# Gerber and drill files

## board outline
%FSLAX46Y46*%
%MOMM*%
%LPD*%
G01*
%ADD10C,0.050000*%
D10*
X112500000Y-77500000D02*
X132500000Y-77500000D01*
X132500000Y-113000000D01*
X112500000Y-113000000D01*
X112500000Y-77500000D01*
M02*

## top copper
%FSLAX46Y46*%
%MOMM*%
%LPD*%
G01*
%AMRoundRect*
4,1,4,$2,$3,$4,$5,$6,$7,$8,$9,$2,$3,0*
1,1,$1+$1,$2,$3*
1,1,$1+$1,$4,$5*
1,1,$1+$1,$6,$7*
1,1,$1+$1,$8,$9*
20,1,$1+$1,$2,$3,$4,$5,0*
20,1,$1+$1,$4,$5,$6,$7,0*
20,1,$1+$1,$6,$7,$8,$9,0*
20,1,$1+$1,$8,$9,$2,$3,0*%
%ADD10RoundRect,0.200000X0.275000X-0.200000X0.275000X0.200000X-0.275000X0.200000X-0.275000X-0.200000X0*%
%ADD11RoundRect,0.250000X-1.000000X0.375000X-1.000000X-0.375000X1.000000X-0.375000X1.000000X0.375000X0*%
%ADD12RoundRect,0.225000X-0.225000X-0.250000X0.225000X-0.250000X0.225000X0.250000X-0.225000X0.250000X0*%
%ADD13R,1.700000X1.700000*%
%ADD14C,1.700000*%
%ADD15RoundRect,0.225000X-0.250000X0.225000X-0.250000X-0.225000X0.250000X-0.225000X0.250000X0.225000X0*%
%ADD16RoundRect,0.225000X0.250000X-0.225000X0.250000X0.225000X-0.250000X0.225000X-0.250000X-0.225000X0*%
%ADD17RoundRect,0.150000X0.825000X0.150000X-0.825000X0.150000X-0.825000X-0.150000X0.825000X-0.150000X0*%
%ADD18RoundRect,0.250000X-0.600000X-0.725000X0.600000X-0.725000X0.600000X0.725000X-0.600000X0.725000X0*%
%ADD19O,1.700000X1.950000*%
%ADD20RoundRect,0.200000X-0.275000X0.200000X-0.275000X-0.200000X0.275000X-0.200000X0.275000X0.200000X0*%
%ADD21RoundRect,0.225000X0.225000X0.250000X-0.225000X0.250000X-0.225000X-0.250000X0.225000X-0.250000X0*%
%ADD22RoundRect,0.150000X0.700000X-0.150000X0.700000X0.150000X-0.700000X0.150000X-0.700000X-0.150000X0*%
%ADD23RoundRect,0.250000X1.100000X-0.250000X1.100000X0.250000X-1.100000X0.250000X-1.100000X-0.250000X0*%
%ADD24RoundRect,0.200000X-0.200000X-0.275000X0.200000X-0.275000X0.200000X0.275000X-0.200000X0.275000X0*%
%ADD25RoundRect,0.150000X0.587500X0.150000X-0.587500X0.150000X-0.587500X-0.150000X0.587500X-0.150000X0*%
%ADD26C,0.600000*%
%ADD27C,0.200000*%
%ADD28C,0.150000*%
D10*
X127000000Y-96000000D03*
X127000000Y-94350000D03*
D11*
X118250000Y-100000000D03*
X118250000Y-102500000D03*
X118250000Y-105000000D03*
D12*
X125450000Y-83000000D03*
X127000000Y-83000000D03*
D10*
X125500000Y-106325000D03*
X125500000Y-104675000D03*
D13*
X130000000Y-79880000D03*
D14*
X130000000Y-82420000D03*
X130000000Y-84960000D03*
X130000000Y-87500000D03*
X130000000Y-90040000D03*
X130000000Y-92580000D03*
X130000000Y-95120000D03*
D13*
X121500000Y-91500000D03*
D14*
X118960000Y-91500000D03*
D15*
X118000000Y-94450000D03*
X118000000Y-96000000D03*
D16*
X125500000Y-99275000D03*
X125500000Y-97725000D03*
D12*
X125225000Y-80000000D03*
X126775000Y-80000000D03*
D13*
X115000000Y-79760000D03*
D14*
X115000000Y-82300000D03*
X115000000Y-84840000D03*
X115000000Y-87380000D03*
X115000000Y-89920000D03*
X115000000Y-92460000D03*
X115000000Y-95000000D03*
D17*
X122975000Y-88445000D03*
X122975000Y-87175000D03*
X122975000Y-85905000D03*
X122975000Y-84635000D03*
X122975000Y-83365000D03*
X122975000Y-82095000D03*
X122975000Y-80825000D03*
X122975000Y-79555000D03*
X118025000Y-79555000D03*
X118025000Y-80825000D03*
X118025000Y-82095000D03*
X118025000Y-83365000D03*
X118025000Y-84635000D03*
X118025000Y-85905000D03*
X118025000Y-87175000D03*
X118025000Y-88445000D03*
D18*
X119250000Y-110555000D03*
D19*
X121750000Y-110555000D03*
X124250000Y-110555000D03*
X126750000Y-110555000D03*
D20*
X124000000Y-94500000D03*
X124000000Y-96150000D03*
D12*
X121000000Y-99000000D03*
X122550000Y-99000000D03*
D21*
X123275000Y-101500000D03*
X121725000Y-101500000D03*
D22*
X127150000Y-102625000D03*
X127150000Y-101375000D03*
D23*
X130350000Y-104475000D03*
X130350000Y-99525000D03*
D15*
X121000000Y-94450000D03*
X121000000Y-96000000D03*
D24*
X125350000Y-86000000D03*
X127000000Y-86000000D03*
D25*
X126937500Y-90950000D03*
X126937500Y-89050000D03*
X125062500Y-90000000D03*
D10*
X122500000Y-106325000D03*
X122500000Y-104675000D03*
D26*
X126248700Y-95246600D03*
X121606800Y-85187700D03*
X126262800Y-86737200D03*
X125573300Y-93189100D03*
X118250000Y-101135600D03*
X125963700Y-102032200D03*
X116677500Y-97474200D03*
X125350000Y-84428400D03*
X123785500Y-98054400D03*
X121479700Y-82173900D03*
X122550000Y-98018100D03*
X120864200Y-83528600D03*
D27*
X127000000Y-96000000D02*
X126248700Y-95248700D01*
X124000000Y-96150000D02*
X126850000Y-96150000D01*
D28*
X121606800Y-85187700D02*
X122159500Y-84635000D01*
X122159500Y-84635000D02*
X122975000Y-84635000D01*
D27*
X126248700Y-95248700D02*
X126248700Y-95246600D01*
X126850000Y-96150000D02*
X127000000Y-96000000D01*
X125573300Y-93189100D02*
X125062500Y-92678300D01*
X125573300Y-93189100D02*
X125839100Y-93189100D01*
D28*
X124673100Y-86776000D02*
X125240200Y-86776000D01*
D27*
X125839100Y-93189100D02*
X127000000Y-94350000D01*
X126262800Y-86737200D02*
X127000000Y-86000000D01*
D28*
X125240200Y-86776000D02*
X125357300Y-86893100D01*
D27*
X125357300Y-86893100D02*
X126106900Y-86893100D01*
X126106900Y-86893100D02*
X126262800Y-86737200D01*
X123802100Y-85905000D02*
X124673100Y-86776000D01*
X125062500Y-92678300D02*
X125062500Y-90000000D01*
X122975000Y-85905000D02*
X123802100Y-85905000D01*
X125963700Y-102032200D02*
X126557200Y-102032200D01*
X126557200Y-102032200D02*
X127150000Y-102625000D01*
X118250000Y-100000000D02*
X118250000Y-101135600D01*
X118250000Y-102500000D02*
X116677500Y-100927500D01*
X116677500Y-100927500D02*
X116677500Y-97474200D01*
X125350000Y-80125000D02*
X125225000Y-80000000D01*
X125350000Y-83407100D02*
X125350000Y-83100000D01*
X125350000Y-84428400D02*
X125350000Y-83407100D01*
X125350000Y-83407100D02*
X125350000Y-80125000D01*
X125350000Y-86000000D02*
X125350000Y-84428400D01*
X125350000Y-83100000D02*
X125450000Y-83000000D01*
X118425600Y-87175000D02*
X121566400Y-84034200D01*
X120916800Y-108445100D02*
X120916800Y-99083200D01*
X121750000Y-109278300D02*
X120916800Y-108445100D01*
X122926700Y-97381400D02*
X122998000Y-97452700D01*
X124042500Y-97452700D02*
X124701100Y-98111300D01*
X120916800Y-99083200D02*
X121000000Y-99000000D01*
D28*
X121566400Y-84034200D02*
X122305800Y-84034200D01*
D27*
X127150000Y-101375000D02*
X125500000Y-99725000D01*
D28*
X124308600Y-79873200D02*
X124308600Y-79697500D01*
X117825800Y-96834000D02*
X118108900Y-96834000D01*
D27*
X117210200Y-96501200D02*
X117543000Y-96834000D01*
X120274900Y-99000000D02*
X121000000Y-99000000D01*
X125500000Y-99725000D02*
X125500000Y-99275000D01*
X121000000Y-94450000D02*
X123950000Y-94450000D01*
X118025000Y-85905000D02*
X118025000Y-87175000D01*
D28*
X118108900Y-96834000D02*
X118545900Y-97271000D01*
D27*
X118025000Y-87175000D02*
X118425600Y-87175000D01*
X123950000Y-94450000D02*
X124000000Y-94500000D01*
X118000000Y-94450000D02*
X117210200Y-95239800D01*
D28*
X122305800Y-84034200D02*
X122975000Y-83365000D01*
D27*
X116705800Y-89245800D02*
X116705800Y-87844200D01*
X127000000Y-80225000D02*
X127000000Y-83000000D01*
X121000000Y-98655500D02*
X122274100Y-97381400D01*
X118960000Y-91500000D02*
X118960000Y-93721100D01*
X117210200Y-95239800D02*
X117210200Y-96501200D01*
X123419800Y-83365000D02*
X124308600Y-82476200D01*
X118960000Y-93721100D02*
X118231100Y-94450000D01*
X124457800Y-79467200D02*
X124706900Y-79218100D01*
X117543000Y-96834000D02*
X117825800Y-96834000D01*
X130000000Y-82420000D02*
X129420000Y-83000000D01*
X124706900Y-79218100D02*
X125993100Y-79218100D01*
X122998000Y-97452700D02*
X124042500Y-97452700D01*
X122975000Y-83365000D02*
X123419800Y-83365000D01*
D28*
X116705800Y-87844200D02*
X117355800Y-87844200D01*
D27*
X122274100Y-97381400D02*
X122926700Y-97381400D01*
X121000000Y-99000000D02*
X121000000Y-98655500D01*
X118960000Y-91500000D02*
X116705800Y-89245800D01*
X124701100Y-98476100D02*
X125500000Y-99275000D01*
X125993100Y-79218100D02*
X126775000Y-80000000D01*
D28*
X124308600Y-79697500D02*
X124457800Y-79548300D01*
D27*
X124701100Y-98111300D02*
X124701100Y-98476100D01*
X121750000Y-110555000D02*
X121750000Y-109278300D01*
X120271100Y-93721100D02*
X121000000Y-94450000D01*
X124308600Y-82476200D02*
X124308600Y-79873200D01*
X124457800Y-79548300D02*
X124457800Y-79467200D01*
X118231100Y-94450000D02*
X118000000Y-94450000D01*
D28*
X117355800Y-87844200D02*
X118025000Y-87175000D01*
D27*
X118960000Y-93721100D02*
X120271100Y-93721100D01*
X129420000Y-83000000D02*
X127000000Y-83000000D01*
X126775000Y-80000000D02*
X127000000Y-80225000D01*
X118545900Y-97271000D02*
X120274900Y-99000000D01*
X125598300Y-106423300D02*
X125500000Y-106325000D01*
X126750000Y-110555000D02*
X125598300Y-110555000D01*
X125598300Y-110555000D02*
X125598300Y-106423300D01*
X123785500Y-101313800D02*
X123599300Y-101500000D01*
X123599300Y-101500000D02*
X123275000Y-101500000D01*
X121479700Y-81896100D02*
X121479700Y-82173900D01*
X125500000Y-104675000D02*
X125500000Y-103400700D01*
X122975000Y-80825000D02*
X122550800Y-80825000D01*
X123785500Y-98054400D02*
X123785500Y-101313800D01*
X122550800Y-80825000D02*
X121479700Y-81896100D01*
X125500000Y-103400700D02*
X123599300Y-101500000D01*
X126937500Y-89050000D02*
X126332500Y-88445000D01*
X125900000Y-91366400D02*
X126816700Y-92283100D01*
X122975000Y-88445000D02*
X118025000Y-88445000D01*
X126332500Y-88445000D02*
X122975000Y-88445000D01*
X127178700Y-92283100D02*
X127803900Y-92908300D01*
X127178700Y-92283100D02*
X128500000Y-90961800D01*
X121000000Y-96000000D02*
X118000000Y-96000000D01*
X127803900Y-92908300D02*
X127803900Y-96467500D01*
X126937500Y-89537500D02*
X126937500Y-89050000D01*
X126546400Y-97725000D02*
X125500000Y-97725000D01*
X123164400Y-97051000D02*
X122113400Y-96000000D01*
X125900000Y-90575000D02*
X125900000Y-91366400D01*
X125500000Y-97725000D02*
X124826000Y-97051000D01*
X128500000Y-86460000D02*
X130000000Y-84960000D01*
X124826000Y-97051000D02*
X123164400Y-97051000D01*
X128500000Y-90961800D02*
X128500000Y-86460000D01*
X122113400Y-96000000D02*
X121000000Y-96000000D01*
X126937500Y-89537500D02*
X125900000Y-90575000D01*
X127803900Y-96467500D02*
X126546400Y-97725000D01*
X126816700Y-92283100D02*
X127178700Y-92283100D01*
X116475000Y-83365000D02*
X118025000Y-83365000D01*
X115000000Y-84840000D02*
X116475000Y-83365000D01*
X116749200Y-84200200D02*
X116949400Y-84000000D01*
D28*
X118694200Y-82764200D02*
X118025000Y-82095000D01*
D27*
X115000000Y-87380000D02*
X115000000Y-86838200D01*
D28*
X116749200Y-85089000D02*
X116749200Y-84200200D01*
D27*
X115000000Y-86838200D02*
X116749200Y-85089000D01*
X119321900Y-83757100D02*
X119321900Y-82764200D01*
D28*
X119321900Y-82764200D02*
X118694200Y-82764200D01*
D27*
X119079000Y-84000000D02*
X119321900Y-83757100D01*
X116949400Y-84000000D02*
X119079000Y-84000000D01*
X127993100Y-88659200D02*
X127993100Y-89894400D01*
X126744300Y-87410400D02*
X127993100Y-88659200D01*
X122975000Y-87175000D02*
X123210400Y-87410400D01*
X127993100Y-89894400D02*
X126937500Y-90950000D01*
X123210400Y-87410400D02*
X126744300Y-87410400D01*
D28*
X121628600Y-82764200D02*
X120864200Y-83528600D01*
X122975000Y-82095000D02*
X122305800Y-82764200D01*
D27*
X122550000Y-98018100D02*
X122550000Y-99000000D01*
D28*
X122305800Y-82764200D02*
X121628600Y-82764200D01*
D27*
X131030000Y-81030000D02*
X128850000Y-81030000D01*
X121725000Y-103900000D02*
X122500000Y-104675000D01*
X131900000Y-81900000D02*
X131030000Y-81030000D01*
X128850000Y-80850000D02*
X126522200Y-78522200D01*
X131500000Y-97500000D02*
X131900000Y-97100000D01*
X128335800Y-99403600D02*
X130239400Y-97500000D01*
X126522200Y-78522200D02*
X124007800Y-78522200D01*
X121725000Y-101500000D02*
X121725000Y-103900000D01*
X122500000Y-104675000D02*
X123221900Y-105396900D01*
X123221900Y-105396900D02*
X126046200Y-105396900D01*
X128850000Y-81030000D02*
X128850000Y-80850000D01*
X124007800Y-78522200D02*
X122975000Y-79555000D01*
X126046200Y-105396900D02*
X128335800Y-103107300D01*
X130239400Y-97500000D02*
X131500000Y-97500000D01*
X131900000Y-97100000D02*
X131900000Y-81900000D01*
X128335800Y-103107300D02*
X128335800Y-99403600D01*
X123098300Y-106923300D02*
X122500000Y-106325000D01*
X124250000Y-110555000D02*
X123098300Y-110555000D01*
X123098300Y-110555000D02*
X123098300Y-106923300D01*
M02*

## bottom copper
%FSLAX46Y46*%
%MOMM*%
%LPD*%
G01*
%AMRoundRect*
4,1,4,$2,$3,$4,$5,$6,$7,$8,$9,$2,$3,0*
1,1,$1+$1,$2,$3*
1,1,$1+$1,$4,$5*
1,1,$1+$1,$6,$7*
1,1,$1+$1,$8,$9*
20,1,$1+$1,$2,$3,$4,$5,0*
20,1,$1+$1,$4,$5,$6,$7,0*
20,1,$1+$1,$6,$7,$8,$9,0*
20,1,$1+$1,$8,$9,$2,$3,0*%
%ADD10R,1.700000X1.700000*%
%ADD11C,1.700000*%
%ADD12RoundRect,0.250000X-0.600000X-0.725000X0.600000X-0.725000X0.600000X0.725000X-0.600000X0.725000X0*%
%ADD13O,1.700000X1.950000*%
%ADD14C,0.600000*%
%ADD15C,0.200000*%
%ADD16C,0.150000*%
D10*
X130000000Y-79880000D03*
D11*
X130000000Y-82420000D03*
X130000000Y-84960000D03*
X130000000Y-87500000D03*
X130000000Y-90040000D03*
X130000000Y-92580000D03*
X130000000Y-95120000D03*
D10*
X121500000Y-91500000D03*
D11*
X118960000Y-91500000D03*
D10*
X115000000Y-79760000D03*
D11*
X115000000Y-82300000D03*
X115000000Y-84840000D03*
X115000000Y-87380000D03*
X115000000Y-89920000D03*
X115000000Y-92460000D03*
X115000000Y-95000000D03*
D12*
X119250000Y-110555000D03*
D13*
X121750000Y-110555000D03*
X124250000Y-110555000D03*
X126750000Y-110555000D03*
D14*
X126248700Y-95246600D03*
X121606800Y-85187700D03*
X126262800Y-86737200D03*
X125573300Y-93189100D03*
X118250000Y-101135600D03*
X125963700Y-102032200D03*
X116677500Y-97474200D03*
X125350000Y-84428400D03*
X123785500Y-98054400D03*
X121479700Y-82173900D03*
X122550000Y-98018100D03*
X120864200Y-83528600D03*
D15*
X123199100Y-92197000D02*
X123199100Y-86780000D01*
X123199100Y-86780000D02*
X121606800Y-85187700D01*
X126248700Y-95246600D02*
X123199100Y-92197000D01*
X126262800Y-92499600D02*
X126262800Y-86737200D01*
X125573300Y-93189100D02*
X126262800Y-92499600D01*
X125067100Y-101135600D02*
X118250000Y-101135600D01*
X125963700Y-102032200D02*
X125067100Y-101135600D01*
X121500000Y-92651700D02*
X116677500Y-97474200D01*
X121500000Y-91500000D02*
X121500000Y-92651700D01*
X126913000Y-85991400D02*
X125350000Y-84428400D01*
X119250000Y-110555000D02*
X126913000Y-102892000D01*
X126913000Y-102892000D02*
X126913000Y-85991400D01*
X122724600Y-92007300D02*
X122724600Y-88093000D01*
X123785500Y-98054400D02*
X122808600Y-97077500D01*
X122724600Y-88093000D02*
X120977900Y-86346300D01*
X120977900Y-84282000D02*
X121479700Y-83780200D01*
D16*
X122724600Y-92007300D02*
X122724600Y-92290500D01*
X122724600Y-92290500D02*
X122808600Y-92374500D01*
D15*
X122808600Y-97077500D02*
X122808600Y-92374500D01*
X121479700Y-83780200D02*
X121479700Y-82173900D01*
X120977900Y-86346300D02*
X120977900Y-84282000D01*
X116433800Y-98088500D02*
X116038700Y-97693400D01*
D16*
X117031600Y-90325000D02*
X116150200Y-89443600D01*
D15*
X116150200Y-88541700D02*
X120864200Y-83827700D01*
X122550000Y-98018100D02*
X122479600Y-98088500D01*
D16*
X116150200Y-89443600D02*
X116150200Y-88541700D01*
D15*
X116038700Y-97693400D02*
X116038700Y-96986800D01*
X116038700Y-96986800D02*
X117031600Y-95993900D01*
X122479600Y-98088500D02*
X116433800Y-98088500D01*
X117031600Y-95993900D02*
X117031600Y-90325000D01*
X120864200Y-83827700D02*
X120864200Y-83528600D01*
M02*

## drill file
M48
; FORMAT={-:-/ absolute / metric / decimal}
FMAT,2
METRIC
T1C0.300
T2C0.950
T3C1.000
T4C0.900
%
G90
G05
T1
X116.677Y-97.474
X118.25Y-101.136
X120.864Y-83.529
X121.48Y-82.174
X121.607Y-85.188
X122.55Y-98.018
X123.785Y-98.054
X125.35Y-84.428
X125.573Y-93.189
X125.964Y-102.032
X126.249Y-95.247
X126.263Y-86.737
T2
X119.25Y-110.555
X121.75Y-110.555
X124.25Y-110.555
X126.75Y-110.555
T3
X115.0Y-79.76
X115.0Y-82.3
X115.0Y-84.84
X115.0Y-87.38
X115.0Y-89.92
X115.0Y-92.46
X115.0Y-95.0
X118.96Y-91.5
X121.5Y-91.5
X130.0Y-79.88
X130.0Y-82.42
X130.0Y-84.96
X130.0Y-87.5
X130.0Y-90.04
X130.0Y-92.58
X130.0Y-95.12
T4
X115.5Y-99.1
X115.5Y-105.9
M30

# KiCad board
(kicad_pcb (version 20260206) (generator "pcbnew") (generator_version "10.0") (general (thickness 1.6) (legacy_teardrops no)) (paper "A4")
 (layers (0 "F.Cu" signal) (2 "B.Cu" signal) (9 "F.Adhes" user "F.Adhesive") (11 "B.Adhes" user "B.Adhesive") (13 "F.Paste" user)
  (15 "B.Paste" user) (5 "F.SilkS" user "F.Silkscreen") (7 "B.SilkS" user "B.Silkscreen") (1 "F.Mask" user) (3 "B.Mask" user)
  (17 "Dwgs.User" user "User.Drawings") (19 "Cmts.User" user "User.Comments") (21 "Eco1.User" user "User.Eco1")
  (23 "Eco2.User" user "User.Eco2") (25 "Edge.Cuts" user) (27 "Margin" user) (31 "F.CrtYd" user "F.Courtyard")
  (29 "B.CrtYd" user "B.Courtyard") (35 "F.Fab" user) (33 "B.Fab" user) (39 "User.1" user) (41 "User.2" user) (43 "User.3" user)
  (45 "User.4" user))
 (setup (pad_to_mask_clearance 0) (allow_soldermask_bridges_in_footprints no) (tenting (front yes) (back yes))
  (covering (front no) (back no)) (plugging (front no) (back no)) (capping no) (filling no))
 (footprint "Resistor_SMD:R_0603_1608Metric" (layer "F.Cu") (at 127 95.175 90)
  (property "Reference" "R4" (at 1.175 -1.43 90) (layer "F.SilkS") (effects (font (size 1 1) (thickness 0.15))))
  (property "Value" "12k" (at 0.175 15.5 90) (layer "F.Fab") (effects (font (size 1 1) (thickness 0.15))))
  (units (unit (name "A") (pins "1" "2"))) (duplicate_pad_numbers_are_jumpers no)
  (pad "1" smd roundrect (at -0.825 0 90) (size 0.8 0.95) (layers "F.Cu" "F.Mask" "F.Paste") (roundrect_rratio 0.25) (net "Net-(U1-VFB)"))
  (pad "2" smd roundrect (at 0.825 0 90) (size 0.8 0.95) (layers "F.Cu" "F.Mask" "F.Paste") (roundrect_rratio 0.25) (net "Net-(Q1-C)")))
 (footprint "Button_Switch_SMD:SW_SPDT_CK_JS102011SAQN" (layer "F.Cu") (at 115.5 102.5 -90)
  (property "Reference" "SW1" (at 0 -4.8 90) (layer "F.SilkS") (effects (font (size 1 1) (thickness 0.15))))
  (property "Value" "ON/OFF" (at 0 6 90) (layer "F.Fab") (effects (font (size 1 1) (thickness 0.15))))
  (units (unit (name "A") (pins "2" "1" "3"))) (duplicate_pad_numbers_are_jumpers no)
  (pad "" np_thru_hole circle (at -3.4 0 270) (size 0.9 0.9) (drill 0.9) (layers "*.Cu" "*.Mask"))
  (pad "" np_thru_hole circle (at 3.4 0 270) (size 0.9 0.9) (drill 0.9) (layers "*.Cu" "*.Mask"))
  (pad "1" smd roundrect (at -2.5 -2.75 270) (size 1.25 2.5) (layers "F.Cu" "F.Mask" "F.Paste") (roundrect_rratio 0.2) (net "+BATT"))
  (pad "2" smd roundrect (at 0 -2.75 270) (size 1.25 2.5) (layers "F.Cu" "F.Mask" "F.Paste") (roundrect_rratio 0.2) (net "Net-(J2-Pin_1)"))
  (pad "3" smd roundrect (at 2.5 -2.75 270) (size 1.25 2.5) (layers "F.Cu" "F.Mask" "F.Paste") (roundrect_rratio 0.2)
   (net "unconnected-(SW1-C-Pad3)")))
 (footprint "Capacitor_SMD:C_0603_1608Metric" (layer "F.Cu") (at 126.225 83)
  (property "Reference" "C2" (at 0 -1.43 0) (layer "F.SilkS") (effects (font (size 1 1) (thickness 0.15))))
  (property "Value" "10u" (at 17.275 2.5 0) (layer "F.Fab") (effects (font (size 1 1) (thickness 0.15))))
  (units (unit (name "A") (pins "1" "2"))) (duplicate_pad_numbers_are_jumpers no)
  (pad "1" smd roundrect (at -0.775 0) (size 0.9 0.95) (layers "F.Cu" "F.Mask" "F.Paste") (roundrect_rratio 0.25) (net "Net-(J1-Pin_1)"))
  (pad "2" smd roundrect (at 0.775 0) (size 0.9 0.95) (layers "F.Cu" "F.Mask" "F.Paste") (roundrect_rratio 0.25) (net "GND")))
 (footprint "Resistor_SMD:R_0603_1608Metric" (layer "F.Cu") (at 125.5 105.5 90)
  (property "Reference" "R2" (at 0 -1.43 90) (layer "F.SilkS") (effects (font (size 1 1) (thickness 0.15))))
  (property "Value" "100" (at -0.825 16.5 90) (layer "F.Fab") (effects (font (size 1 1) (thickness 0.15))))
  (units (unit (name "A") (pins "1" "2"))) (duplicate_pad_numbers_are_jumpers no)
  (pad "1" smd roundrect (at -0.825 0 90) (size 0.8 0.95) (layers "F.Cu" "F.Mask" "F.Paste") (roundrect_rratio 0.25) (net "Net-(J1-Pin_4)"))
  (pad "2" smd roundrect (at 0.825 0 90) (size 0.8 0.95) (layers "F.Cu" "F.Mask" "F.Paste") (roundrect_rratio 0.25) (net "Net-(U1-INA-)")))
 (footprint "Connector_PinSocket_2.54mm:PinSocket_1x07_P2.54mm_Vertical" (layer "F.Cu") (at 130 79.88)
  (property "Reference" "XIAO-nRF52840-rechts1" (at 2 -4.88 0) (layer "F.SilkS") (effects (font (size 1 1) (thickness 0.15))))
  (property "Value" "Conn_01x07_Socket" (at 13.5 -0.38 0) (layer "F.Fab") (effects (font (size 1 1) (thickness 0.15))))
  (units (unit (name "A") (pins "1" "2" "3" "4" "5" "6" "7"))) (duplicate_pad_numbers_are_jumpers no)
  (pad "1" thru_hole rect (at 0 0) (size 1.7 1.7) (drill 1) (layers "*.Cu" "*.Mask") (remove_unused_layers no)
   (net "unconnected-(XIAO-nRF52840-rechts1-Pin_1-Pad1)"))
  (pad "2" thru_hole circle (at 0 2.54) (size 1.7 1.7) (drill 1) (layers "*.Cu" "*.Mask") (remove_unused_layers no) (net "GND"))
  (pad "3" thru_hole circle (at 0 5.08) (size 1.7 1.7) (drill 1) (layers "*.Cu" "*.Mask") (remove_unused_layers no) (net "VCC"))
  (pad "4" thru_hole circle (at 0 7.62) (size 1.7 1.7) (drill 1) (layers "*.Cu" "*.Mask") (remove_unused_layers no)
   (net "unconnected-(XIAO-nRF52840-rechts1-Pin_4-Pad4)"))
  (pad "5" thru_hole circle (at 0 10.16) (size 1.7 1.7) (drill 1) (layers "*.Cu" "*.Mask") (remove_unused_layers no)
   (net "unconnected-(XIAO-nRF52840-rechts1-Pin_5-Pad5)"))
  (pad "6" thru_hole circle (at 0 12.7) (size 1.7 1.7) (drill 1) (layers "*.Cu" "*.Mask") (remove_unused_layers no)
   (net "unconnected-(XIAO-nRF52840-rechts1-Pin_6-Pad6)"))
  (pad "7" thru_hole circle (at 0 15.24) (size 1.7 1.7) (drill 1) (layers "*.Cu" "*.Mask") (remove_unused_layers no)
   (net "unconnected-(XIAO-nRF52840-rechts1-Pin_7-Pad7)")))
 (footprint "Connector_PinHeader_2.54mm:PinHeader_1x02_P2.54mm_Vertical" (layer "F.Cu") (at 121.5 91.5 -90)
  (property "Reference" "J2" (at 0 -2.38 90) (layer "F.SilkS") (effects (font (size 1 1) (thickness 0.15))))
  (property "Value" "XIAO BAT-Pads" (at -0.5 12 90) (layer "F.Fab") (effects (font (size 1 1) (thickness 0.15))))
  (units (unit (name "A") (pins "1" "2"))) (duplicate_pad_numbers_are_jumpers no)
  (pad "1" thru_hole rect (at 0 0 270) (size 1.7 1.7) (drill 1) (layers "*.Cu" "*.Mask") (remove_unused_layers no) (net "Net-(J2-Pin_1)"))
  (pad "2" thru_hole circle (at 0 2.54 270) (size 1.7 1.7) (drill 1) (layers "*.Cu" "*.Mask") (remove_unused_layers no) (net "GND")))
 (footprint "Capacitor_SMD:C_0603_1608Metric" (layer "F.Cu") (at 118 95.225 -90)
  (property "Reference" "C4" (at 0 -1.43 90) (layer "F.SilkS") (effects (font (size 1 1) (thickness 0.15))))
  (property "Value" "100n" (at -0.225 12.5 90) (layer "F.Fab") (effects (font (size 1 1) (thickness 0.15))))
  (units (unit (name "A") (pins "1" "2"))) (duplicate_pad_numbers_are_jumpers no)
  (pad "1" smd roundrect (at -0.775 0 270) (size 0.9 0.95) (layers "F.Cu" "F.Mask" "F.Paste") (roundrect_rratio 0.25) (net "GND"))
  (pad "2" smd roundrect (at 0.775 0 270) (size 0.9 0.95) (layers "F.Cu" "F.Mask" "F.Paste") (roundrect_rratio 0.25) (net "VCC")))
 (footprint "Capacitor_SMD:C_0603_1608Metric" (layer "F.Cu") (at 125.5 98.5 90)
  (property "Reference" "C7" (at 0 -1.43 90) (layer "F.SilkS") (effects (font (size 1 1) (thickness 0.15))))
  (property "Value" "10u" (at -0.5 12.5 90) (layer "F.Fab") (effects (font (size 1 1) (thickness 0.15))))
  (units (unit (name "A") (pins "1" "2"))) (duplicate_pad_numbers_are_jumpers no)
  (pad "1" smd roundrect (at -0.775 0 90) (size 0.9 0.95) (layers "F.Cu" "F.Mask" "F.Paste") (roundrect_rratio 0.25) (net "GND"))
  (pad "2" smd roundrect (at 0.775 0 90) (size 0.9 0.95) (layers "F.Cu" "F.Mask" "F.Paste") (roundrect_rratio 0.25) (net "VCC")))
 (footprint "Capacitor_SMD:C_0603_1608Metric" (layer "F.Cu") (at 126 80)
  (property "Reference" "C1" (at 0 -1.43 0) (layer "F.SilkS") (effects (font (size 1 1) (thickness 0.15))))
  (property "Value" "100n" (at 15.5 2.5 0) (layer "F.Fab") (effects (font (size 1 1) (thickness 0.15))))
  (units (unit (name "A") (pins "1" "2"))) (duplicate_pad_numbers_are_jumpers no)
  (pad "1" smd roundrect (at -0.775 0) (size 0.9 0.95) (layers "F.Cu" "F.Mask" "F.Paste") (roundrect_rratio 0.25) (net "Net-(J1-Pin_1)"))
  (pad "2" smd roundrect (at 0.775 0) (size 0.9 0.95) (layers "F.Cu" "F.Mask" "F.Paste") (roundrect_rratio 0.25) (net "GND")))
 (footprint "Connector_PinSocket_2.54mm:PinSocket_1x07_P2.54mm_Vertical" (layer "F.Cu") (at 115 79.76)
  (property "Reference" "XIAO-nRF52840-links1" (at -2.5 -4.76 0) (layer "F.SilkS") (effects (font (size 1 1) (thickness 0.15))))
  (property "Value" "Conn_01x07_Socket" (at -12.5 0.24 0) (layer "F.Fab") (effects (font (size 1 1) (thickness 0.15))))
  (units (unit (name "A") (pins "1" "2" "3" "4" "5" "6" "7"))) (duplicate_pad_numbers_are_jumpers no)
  (pad "1" thru_hole rect (at 0 0) (size 1.7 1.7) (drill 1) (layers "*.Cu" "*.Mask") (remove_unused_layers no)
   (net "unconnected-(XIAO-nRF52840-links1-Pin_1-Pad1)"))
  (pad "2" thru_hole circle (at 0 2.54) (size 1.7 1.7) (drill 1) (layers "*.Cu" "*.Mask") (remove_unused_layers no)
   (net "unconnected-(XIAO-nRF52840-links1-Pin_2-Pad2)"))
  (pad "3" thru_hole circle (at 0 5.08) (size 1.7 1.7) (drill 1) (layers "*.Cu" "*.Mask") (remove_unused_layers no) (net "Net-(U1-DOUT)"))
  (pad "4" thru_hole circle (at 0 7.62) (size 1.7 1.7) (drill 1) (layers "*.Cu" "*.Mask") (remove_unused_layers no) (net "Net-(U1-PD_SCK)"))
  (pad "5" thru_hole circle (at 0 10.16) (size 1.7 1.7) (drill 1) (layers "*.Cu" "*.Mask") (remove_unused_layers no)
   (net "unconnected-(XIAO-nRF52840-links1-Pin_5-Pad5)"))
  (pad "6" thru_hole circle (at 0 12.7) (size 1.7 1.7) (drill 1) (layers "*.Cu" "*.Mask") (remove_unused_layers no)
   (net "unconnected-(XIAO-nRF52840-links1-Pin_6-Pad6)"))
  (pad "7" thru_hole circle (at 0 15.24) (size 1.7 1.7) (drill 1) (layers "*.Cu" "*.Mask") (remove_unused_layers no)
   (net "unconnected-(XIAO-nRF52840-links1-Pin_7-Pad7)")))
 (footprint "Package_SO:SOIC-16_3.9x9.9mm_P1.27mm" (layer "F.Cu") (at 120.5 84 180)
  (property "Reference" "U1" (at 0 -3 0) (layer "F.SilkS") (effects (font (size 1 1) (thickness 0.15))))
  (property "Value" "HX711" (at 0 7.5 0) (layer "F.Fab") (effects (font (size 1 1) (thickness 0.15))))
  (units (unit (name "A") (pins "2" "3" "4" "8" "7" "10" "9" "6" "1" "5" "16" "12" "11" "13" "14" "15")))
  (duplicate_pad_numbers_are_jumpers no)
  (pad "1" smd roundrect (at -2.475 -4.445 180) (size 1.95 0.6) (layers "F.Cu" "F.Mask" "F.Paste") (roundrect_rratio 0.25) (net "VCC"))
  (pad "2" smd roundrect (at -2.475 -3.175 180) (size 1.95 0.6) (layers "F.Cu" "F.Mask" "F.Paste") (roundrect_rratio 0.25)
   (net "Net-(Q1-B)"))
  (pad "3" smd roundrect (at -2.475 -1.905 180) (size 1.95 0.6) (layers "F.Cu" "F.Mask" "F.Paste") (roundrect_rratio 0.25)
   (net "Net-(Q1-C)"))
  (pad "4" smd roundrect (at -2.475 -0.635 180) (size 1.95 0.6) (layers "F.Cu" "F.Mask" "F.Paste") (roundrect_rratio 0.25)
   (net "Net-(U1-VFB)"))
  (pad "5" smd roundrect (at -2.475 0.635 180) (size 1.95 0.6) (layers "F.Cu" "F.Mask" "F.Paste") (roundrect_rratio 0.25) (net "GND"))
  (pad "6" smd roundrect (at -2.475 1.905 180) (size 1.95 0.6) (layers "F.Cu" "F.Mask" "F.Paste") (roundrect_rratio 0.25)
   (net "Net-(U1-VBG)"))
  (pad "7" smd roundrect (at -2.475 3.175 180) (size 1.95 0.6) (layers "F.Cu" "F.Mask" "F.Paste") (roundrect_rratio 0.25)
   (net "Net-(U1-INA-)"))
  (pad "8" smd roundrect (at -2.475 4.445 180) (size 1.95 0.6) (layers "F.Cu" "F.Mask" "F.Paste") (roundrect_rratio 0.25)
   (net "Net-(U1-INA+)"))
  (pad "9" smd roundrect (at 2.475 4.445 180) (size 1.95 0.6) (layers "F.Cu" "F.Mask" "F.Paste") (roundrect_rratio 0.25)
   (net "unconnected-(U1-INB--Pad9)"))
  (pad "10" smd roundrect (at 2.475 3.175 180) (size 1.95 0.6) (layers "F.Cu" "F.Mask" "F.Paste") (roundrect_rratio 0.25)
   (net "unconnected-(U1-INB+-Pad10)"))
  (pad "11" smd roundrect (at 2.475 1.905 180) (size 1.95 0.6) (layers "F.Cu" "F.Mask" "F.Paste") (roundrect_rratio 0.25)
   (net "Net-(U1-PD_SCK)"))
  (pad "12" smd roundrect (at 2.475 0.635 180) (size 1.95 0.6) (layers "F.Cu" "F.Mask" "F.Paste") (roundrect_rratio 0.25)
   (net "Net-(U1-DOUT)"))
  (pad "13" smd roundrect (at 2.475 -0.635 180) (size 1.95 0.6) (layers "F.Cu" "F.Mask" "F.Paste") (roundrect_rratio 0.25)
   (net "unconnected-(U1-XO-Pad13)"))
  (pad "14" smd roundrect (at 2.475 -1.905 180) (size 1.95 0.6) (layers "F.Cu" "F.Mask" "F.Paste") (roundrect_rratio 0.25) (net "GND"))
  (pad "15" smd roundrect (at 2.475 -3.175 180) (size 1.95 0.6) (layers "F.Cu" "F.Mask" "F.Paste") (roundrect_rratio 0.25) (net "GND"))
  (pad "16" smd roundrect (at 2.475 -4.445 180) (size 1.95 0.6) (layers "F.Cu" "F.Mask" "F.Paste") (roundrect_rratio 0.25) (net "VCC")))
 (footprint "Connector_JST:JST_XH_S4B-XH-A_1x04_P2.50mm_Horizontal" (layer "F.Cu") (at 119.25 110.555)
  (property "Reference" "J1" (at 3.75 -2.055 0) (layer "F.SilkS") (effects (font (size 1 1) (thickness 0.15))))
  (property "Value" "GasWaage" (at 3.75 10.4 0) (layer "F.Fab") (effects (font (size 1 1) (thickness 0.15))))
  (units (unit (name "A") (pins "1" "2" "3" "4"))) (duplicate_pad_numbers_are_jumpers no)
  (pad "1" thru_hole roundrect (at 0 0) (size 1.7 1.95) (drill 0.95) (layers "*.Cu" "*.Mask") (remove_unused_layers no)
   (roundrect_rratio 0.147059) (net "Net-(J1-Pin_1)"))
  (pad "2" thru_hole oval (at 2.5 0) (size 1.7 1.95) (drill 0.95) (layers "*.Cu" "*.Mask") (remove_unused_layers no) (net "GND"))
  (pad "3" thru_hole oval (at 5 0) (size 1.7 1.95) (drill 0.95) (layers "*.Cu" "*.Mask") (remove_unused_layers no) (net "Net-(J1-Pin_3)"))
  (pad "4" thru_hole oval (at 7.5 0) (size 1.7 1.95) (drill 0.95) (layers "*.Cu" "*.Mask") (remove_unused_layers no) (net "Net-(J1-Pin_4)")))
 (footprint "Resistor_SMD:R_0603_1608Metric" (layer "F.Cu") (at 124 95.325 -90)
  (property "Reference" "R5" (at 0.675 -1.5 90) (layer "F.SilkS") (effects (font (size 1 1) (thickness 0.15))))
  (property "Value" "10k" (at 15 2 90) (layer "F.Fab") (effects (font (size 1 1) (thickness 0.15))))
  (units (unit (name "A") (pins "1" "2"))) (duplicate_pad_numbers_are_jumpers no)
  (pad "1" smd roundrect (at -0.825 0 270) (size 0.8 0.95) (layers "F.Cu" "F.Mask" "F.Paste") (roundrect_rratio 0.25) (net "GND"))
  (pad "2" smd roundrect (at 0.825 0 270) (size 0.8 0.95) (layers "F.Cu" "F.Mask" "F.Paste") (roundrect_rratio 0.25) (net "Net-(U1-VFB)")))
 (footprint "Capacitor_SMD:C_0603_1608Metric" (layer "F.Cu") (at 121.775 99)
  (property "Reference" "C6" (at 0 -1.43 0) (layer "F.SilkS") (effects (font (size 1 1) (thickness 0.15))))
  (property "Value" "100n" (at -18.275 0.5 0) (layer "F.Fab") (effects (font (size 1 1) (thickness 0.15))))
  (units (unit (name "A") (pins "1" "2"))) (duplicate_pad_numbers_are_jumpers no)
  (pad "1" smd roundrect (at -0.775 0) (size 0.9 0.95) (layers "F.Cu" "F.Mask" "F.Paste") (roundrect_rratio 0.25) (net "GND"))
  (pad "2" smd roundrect (at 0.775 0) (size 0.9 0.95) (layers "F.Cu" "F.Mask" "F.Paste") (roundrect_rratio 0.25) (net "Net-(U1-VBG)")))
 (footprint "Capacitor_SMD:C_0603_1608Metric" (layer "F.Cu") (at 122.5 101.5 180)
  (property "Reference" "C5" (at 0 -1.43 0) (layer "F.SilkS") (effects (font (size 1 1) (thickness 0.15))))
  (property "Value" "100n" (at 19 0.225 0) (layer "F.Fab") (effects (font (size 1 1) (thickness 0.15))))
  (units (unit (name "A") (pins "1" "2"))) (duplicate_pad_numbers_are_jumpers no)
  (pad "1" smd roundrect (at -0.775 0 180) (size 0.9 0.95) (layers "F.Cu" "F.Mask" "F.Paste") (roundrect_rratio 0.25) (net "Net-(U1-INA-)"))
  (pad "2" smd roundrect (at 0.775 0 180) (size 0.9 0.95) (layers "F.Cu" "F.Mask" "F.Paste") (roundrect_rratio 0.25) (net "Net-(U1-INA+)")))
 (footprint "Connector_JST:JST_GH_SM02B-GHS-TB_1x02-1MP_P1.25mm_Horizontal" (layer "F.Cu") (at 129 102 90)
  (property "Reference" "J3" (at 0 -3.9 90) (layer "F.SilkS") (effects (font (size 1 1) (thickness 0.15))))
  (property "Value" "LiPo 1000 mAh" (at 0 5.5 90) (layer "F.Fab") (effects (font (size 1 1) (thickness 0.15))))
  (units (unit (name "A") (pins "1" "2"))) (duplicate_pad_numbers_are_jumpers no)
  (pad "1" smd roundrect (at -0.625 -1.85 90) (size 0.6 1.7) (layers "F.Cu" "F.Mask" "F.Paste") (roundrect_rratio 0.25) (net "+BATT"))
  (pad "2" smd roundrect (at 0.625 -1.85 90) (size 0.6 1.7) (layers "F.Cu" "F.Mask" "F.Paste") (roundrect_rratio 0.25) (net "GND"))
  (pad "MP" smd roundrect (at -2.475 1.35 90) (size 1 2.7) (layers "F.Cu" "F.Mask" "F.Paste") (roundrect_rratio 0.25))
  (pad "MP" smd roundrect (at 2.475 1.35 90) (size 1 2.7) (layers "F.Cu" "F.Mask" "F.Paste") (roundrect_rratio 0.25)))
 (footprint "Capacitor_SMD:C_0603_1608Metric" (layer "F.Cu") (at 121 95.225 -90)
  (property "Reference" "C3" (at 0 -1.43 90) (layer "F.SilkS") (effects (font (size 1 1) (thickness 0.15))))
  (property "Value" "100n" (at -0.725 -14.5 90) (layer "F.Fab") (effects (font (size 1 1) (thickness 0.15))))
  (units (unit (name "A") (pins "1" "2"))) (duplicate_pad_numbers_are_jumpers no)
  (pad "1" smd roundrect (at -0.775 0 270) (size 0.9 0.95) (layers "F.Cu" "F.Mask" "F.Paste") (roundrect_rratio 0.25) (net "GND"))
  (pad "2" smd roundrect (at 0.775 0 270) (size 0.9 0.95) (layers "F.Cu" "F.Mask" "F.Paste") (roundrect_rratio 0.25) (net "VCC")))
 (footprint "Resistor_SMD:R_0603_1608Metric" (layer "F.Cu") (at 126.175 86)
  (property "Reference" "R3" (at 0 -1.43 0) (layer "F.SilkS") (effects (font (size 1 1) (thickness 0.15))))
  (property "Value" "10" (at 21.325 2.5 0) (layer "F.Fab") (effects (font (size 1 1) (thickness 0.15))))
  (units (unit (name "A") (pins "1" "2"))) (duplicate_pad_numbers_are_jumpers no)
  (pad "1" smd roundrect (at -0.825 0) (size 0.8 0.95) (layers "F.Cu" "F.Mask" "F.Paste") (roundrect_rratio 0.25) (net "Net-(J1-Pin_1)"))
  (pad "2" smd roundrect (at 0.825 0) (size 0.8 0.95) (layers "F.Cu" "F.Mask" "F.Paste") (roundrect_rratio 0.25) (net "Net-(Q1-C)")))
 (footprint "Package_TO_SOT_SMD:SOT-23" (layer "F.Cu") (at 126 90 180)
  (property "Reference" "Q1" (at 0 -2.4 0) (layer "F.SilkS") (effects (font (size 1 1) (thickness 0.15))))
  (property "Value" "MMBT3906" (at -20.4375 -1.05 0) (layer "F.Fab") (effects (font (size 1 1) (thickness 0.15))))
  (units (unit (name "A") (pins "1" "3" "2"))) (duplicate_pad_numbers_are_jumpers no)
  (pad "1" smd roundrect (at -0.9375 -0.95 180) (size 1.475 0.6) (layers "F.Cu" "F.Mask" "F.Paste") (roundrect_rratio 0.25)
   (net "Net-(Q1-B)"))
  (pad "2" smd roundrect (at -0.9375 0.95 180) (size 1.475 0.6) (layers "F.Cu" "F.Mask" "F.Paste") (roundrect_rratio 0.25) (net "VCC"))
  (pad "3" smd roundrect (at 0.9375 0 180) (size 1.475 0.6) (layers "F.Cu" "F.Mask" "F.Paste") (roundrect_rratio 0.25) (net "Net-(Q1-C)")))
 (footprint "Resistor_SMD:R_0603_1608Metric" (layer "F.Cu") (at 122.5 105.5 90)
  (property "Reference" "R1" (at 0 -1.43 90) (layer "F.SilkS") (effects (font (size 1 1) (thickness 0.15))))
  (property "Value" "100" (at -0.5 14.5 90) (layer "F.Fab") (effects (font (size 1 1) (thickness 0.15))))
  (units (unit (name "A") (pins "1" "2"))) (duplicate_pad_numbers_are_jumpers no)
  (pad "1" smd roundrect (at -0.825 0 90) (size 0.8 0.95) (layers "F.Cu" "F.Mask" "F.Paste") (roundrect_rratio 0.25) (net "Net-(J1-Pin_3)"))
  (pad "2" smd roundrect (at 0.825 0 90) (size 0.8 0.95) (layers "F.Cu" "F.Mask" "F.Paste") (roundrect_rratio 0.25) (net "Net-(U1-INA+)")))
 (gr_rect (start 112.5 77.5) (end 132.5 113) (stroke (width 0.05) (type solid)) (fill no) (layer "Edge.Cuts"))
 (segment (start 127 96) (end 126.2487 95.2487) (width 0.2) (layer "F.Cu") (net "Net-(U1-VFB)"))
 (segment (start 124 96.15) (end 126.85 96.15) (width 0.2) (layer "F.Cu") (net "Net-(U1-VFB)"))
 (segment (start 121.6068 85.1877) (end 122.1595 84.635) (width 0.15) (layer "F.Cu") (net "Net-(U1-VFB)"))
 (segment (start 122.1595 84.635) (end 122.975 84.635) (width 0.15) (layer "F.Cu") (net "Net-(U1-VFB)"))
 (segment (start 126.2487 95.2487) (end 126.2487 95.2466) (width 0.2) (layer "F.Cu") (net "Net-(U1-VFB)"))
 (segment (start 126.85 96.15) (end 127 96) (width 0.2) (layer "F.Cu") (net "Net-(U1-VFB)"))
 (via (at 126.2487 95.2466) (size 0.6) (drill 0.3) (layers "F.Cu" "B.Cu") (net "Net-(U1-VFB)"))
 (via (at 121.6068 85.1877) (size 0.6) (drill 0.3) (layers "F.Cu" "B.Cu") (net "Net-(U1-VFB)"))
 (segment (start 123.1991 92.197) (end 123.1991 86.78) (width 0.2) (layer "B.Cu") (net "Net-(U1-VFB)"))
 (segment (start 123.1991 86.78) (end 121.6068 85.1877) (width 0.2) (layer "B.Cu") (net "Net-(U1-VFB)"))
 (segment (start 126.2487 95.2466) (end 123.1991 92.197) (width 0.2) (layer "B.Cu") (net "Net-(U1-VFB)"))
 (segment (start 125.5733 93.1891) (end 125.0625 92.6783) (width 0.2) (layer "F.Cu") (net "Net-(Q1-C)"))
 (segment (start 125.5733 93.1891) (end 125.8391 93.1891) (width 0.2) (layer "F.Cu") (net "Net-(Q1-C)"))
 (segment (start 124.6731 86.776) (end 125.2402 86.776) (width 0.15) (layer "F.Cu") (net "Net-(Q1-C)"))
 (segment (start 125.8391 93.1891) (end 127 94.35) (width 0.2) (layer "F.Cu") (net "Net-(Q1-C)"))
 (segment (start 126.2628 86.7372) (end 127 86) (width 0.2) (layer "F.Cu") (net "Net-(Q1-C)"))
 (segment (start 125.2402 86.776) (end 125.3573 86.8931) (width 0.15) (layer "F.Cu") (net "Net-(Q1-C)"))
 (segment (start 125.3573 86.8931) (end 126.1069 86.8931) (width 0.2) (layer "F.Cu") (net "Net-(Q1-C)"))
 (segment (start 126.1069 86.8931) (end 126.2628 86.7372) (width 0.2) (layer "F.Cu") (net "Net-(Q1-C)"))
 (segment (start 123.8021 85.905) (end 124.6731 86.776) (width 0.2) (layer "F.Cu") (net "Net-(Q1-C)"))
 (segment (start 125.0625 92.6783) (end 125.0625 90) (width 0.2) (layer "F.Cu") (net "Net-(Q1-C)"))
 (segment (start 122.975 85.905) (end 123.8021 85.905) (width 0.2) (layer "F.Cu") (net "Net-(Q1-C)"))
 (via (at 126.2628 86.7372) (size 0.6) (drill 0.3) (layers "F.Cu" "B.Cu") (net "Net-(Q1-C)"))
 (via (at 125.5733 93.1891) (size 0.6) (drill 0.3) (layers "F.Cu" "B.Cu") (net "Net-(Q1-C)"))
 (segment (start 126.2628 92.4996) (end 126.2628 86.7372) (width 0.2) (layer "B.Cu") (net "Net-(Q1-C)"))
 (segment (start 125.5733 93.1891) (end 126.2628 92.4996) (width 0.2) (layer "B.Cu") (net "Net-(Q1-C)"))
 (segment (start 125.9637 102.0322) (end 126.5572 102.0322) (width 0.2) (layer "F.Cu") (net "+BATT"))
 (segment (start 126.5572 102.0322) (end 127.15 102.625) (width 0.2) (layer "F.Cu") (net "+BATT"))
 (segment (start 118.25 100) (end 118.25 101.1356) (width 0.2) (layer "F.Cu") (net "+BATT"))
 (via (at 118.25 101.1356) (size 0.6) (drill 0.3) (layers "F.Cu" "B.Cu") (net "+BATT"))
 (via (at 125.9637 102.0322) (size 0.6) (drill 0.3) (layers "F.Cu" "B.Cu") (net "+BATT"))
 (segment (start 125.0671 101.1356) (end 118.25 101.1356) (width 0.2) (layer "B.Cu") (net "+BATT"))
 (segment (start 125.9637 102.0322) (end 125.0671 101.1356) (width 0.2) (layer "B.Cu") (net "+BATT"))
 (segment (start 118.25 102.5) (end 116.6775 100.9275) (width 0.2) (layer "F.Cu") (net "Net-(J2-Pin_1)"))
 (segment (start 116.6775 100.9275) (end 116.6775 97.4742) (width 0.2) (layer "F.Cu") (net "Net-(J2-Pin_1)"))
 (via (at 116.6775 97.4742) (size 0.6) (drill 0.3) (layers "F.Cu" "B.Cu") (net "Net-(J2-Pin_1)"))
 (segment (start 121.5 92.6517) (end 116.6775 97.4742) (width 0.2) (layer "B.Cu") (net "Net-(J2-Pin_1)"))
 (segment (start 121.5 91.5) (end 121.5 92.6517) (width 0.2) (layer "B.Cu") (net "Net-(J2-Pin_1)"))
 (segment (start 125.35 80.125) (end 125.225 80) (width 0.2) (layer "F.Cu") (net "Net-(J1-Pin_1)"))
 (segment (start 125.35 83.4071) (end 125.35 83.1) (width 0.2) (layer "F.Cu") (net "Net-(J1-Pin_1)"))
 (segment (start 125.35 84.4284) (end 125.35 83.4071) (width 0.2) (layer "F.Cu") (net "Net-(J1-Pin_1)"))
 (segment (start 125.35 83.4071) (end 125.35 80.125) (width 0.2) (layer "F.Cu") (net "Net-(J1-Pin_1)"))
 (segment (start 125.35 86) (end 125.35 84.4284) (width 0.2) (layer "F.Cu") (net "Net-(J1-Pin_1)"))
 (segment (start 125.35 83.1) (end 125.45 83) (width 0.2) (layer "F.Cu") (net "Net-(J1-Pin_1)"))
 (via (at 125.35 84.4284) (size 0.6) (drill 0.3) (layers "F.Cu" "B.Cu") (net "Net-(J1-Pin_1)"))
 (segment (start 126.913 85.9914) (end 125.35 84.4284) (width 0.2) (layer "B.Cu") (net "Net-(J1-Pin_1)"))
 (segment (start 119.25 110.555) (end 126.913 102.892) (width 0.2) (layer "B.Cu") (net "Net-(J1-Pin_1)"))
 (segment (start 126.913 102.892) (end 126.913 85.9914) (width 0.2) (layer "B.Cu") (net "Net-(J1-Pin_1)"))
 (segment (start 118.4256 87.175) (end 121.5664 84.0342) (width 0.2) (layer "F.Cu") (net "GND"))
 (segment (start 120.9168 108.4451) (end 120.9168 99.0832) (width 0.2) (layer "F.Cu") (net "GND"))
 (segment (start 121.75 109.2783) (end 120.9168 108.4451) (width 0.2) (layer "F.Cu") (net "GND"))
 (segment (start 122.9267 97.3814) (end 122.998 97.4527) (width 0.2) (layer "F.Cu") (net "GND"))
 (segment (start 124.0425 97.4527) (end 124.7011 98.1113) (width 0.2) (layer "F.Cu") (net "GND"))
 (segment (start 120.9168 99.0832) (end 121 99) (width 0.2) (layer "F.Cu") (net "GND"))
 (segment (start 121.5664 84.0342) (end 122.3058 84.0342) (width 0.15) (layer "F.Cu") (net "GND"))
 (segment (start 127.15 101.375) (end 125.5 99.725) (width 0.2) (layer "F.Cu") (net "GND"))
 (segment (start 124.3086 79.8732) (end 124.3086 79.6975) (width 0.15) (layer "F.Cu") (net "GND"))
 (segment (start 117.8258 96.834) (end 118.1089 96.834) (width 0.15) (layer "F.Cu") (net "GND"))
 (segment (start 117.2102 96.5012) (end 117.543 96.834) (width 0.2) (layer "F.Cu") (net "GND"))
 (segment (start 120.2749 99) (end 121 99) (width 0.2) (layer "F.Cu") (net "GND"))
 (segment (start 125.5 99.725) (end 125.5 99.275) (width 0.2) (layer "F.Cu") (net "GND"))
 (segment (start 121 94.45) (end 123.95 94.45) (width 0.2) (layer "F.Cu") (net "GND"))
 (segment (start 118.025 85.905) (end 118.025 87.175) (width 0.2) (layer "F.Cu") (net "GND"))
 (segment (start 118.1089 96.834) (end 118.5459 97.271) (width 0.15) (layer "F.Cu") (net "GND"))
 (segment (start 118.025 87.175) (end 118.4256 87.175) (width 0.2) (layer "F.Cu") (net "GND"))
 (segment (start 123.95 94.45) (end 124 94.5) (width 0.2) (layer "F.Cu") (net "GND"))
 (segment (start 118 94.45) (end 117.2102 95.2398) (width 0.2) (layer "F.Cu") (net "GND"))
 (segment (start 122.3058 84.0342) (end 122.975 83.365) (width 0.15) (layer "F.Cu") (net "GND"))
 (segment (start 116.7058 89.2458) (end 116.7058 87.8442) (width 0.2) (layer "F.Cu") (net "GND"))
 (segment (start 127 80.225) (end 127 83) (width 0.2) (layer "F.Cu") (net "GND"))
 (segment (start 121 98.6555) (end 122.2741 97.3814) (width 0.2) (layer "F.Cu") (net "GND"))
 (segment (start 118.96 91.5) (end 118.96 93.7211) (width 0.2) (layer "F.Cu") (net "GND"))
 (segment (start 117.2102 95.2398) (end 117.2102 96.5012) (width 0.2) (layer "F.Cu") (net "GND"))
 (segment (start 123.4198 83.365) (end 124.3086 82.4762) (width 0.2) (layer "F.Cu") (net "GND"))
 (segment (start 118.96 93.7211) (end 118.2311 94.45) (width 0.2) (layer "F.Cu") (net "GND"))
 (segment (start 124.4578 79.4672) (end 124.7069 79.2181) (width 0.2) (layer "F.Cu") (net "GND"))
 (segment (start 117.543 96.834) (end 117.8258 96.834) (width 0.2) (layer "F.Cu") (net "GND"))
 (segment (start 130 82.42) (end 129.42 83) (width 0.2) (layer "F.Cu") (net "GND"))
 (segment (start 124.7069 79.2181) (end 125.9931 79.2181) (width 0.2) (layer "F.Cu") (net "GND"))
 (segment (start 122.998 97.4527) (end 124.0425 97.4527) (width 0.2) (layer "F.Cu") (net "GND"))
 (segment (start 122.975 83.365) (end 123.4198 83.365) (width 0.2) (layer "F.Cu") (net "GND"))
 (segment (start 116.7058 87.8442) (end 117.3558 87.8442) (width 0.15) (layer "F.Cu") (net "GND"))
 (segment (start 122.2741 97.3814) (end 122.9267 97.3814) (width 0.2) (layer "F.Cu") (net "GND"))
 (segment (start 121 99) (end 121 98.6555) (width 0.2) (layer "F.Cu") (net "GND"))
 (segment (start 118.96 91.5) (end 116.7058 89.2458) (width 0.2) (layer "F.Cu") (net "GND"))
 (segment (start 124.7011 98.4761) (end 125.5 99.275) (width 0.2) (layer "F.Cu") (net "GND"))
 (segment (start 125.9931 79.2181) (end 126.775 80) (width 0.2) (layer "F.Cu") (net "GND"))
 (segment (start 124.3086 79.6975) (end 124.4578 79.5483) (width 0.15) (layer "F.Cu") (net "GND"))
 (segment (start 124.7011 98.1113) (end 124.7011 98.4761) (width 0.2) (layer "F.Cu") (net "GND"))
 (segment (start 121.75 110.555) (end 121.75 109.2783) (width 0.2) (layer "F.Cu") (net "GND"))
 (segment (start 120.2711 93.7211) (end 121 94.45) (width 0.2) (layer "F.Cu") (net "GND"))
 (segment (start 124.3086 82.4762) (end 124.3086 79.8732) (width 0.2) (layer "F.Cu") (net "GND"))
 (segment (start 124.4578 79.5483) (end 124.4578 79.4672) (width 0.2) (layer "F.Cu") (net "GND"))
 (segment (start 118.2311 94.45) (end 118 94.45) (width 0.2) (layer "F.Cu") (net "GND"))
 (segment (start 117.3558 87.8442) (end 118.025 87.175) (width 0.15) (layer "F.Cu") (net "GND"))
 (segment (start 118.96 93.7211) (end 120.2711 93.7211) (width 0.2) (layer "F.Cu") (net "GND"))
 (segment (start 129.42 83) (end 127 83) (width 0.2) (layer "F.Cu") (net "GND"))
 (segment (start 126.775 80) (end 127 80.225) (width 0.2) (layer "F.Cu") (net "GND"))
 (segment (start 118.5459 97.271) (end 120.2749 99) (width 0.2) (layer "F.Cu") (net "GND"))
 (segment (start 125.5983 106.4233) (end 125.5 106.325) (width 0.2) (layer "F.Cu") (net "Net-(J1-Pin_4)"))
 (segment (start 126.75 110.555) (end 125.5983 110.555) (width 0.2) (layer "F.Cu") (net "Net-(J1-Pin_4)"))
 (segment (start 125.5983 110.555) (end 125.5983 106.4233) (width 0.2) (layer "F.Cu") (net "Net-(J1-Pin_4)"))
 (segment (start 123.7855 101.3138) (end 123.5993 101.5) (width 0.2) (layer "F.Cu") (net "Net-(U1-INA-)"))
 (segment (start 123.5993 101.5) (end 123.275 101.5) (width 0.2) (layer "F.Cu") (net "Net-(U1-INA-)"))
 (segment (start 121.4797 81.8961) (end 121.4797 82.1739) (width 0.2) (layer "F.Cu") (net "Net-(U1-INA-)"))
 (segment (start 125.5 104.675) (end 125.5 103.4007) (width 0.2) (layer "F.Cu") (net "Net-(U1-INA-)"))
 (segment (start 122.975 80.825) (end 122.5508 80.825) (width 0.2) (layer "F.Cu") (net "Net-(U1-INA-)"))
 (segment (start 123.7855 98.0544) (end 123.7855 101.3138) (width 0.2) (layer "F.Cu") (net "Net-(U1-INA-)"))
 (segment (start 122.5508 80.825) (end 121.4797 81.8961) (width 0.2) (layer "F.Cu") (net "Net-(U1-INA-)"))
 (segment (start 125.5 103.4007) (end 123.5993 101.5) (width 0.2) (layer "F.Cu") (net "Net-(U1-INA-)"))
 (via (at 123.7855 98.0544) (size 0.6) (drill 0.3) (layers "F.Cu" "B.Cu") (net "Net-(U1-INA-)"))
 (via (at 121.4797 82.1739) (size 0.6) (drill 0.3) (layers "F.Cu" "B.Cu") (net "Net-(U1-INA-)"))
 (segment (start 122.7246 92.0073) (end 122.7246 88.093) (width 0.2) (layer "B.Cu") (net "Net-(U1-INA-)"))
 (segment (start 123.7855 98.0544) (end 122.8086 97.0775) (width 0.2) (layer "B.Cu") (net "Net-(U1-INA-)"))
 (segment (start 122.7246 88.093) (end 120.9779 86.3463) (width 0.2) (layer "B.Cu") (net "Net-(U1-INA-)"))
 (segment (start 120.9779 84.282) (end 121.4797 83.7802) (width 0.2) (layer "B.Cu") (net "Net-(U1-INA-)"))
 (segment (start 122.7246 92.0073) (end 122.7246 92.2905) (width 0.15) (layer "B.Cu") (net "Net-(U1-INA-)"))
 (segment (start 122.7246 92.2905) (end 122.8086 92.3745) (width 0.15) (layer "B.Cu") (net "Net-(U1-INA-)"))
 (segment (start 122.8086 97.0775) (end 122.8086 92.3745) (width 0.2) (layer "B.Cu") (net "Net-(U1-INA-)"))
 (segment (start 121.4797 83.7802) (end 121.4797 82.1739) (width 0.2) (layer "B.Cu") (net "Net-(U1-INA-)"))
 (segment (start 120.9779 86.3463) (end 120.9779 84.282) (width 0.2) (layer "B.Cu") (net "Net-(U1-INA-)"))
 (segment (start 126.9375 89.05) (end 126.3325 88.445) (width 0.2) (layer "F.Cu") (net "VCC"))
 (segment (start 125.9 91.3664) (end 126.8167 92.2831) (width 0.2) (layer "F.Cu") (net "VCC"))
 (segment (start 122.975 88.445) (end 118.025 88.445) (width 0.2) (layer "F.Cu") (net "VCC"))
 (segment (start 126.3325 88.445) (end 122.975 88.445) (width 0.2) (layer "F.Cu") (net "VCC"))
 (segment (start 127.1787 92.2831) (end 127.8039 92.9083) (width 0.2) (layer "F.Cu") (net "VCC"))
 (segment (start 127.1787 92.2831) (end 128.5 90.9618) (width 0.2) (layer "F.Cu") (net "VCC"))
 (segment (start 121 96) (end 118 96) (width 0.2) (layer "F.Cu") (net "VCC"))
 (segment (start 127.8039 92.9083) (end 127.8039 96.4675) (width 0.2) (layer "F.Cu") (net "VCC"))
 (segment (start 126.9375 89.5375) (end 126.9375 89.05) (width 0.2) (layer "F.Cu") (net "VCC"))
 (segment (start 126.5464 97.725) (end 125.5 97.725) (width 0.2) (layer "F.Cu") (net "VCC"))
 (segment (start 123.1644 97.051) (end 122.1134 96) (width 0.2) (layer "F.Cu") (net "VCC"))
 (segment (start 125.9 90.575) (end 125.9 91.3664) (width 0.2) (layer "F.Cu") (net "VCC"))
 (segment (start 125.5 97.725) (end 124.826 97.051) (width 0.2) (layer "F.Cu") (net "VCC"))
 (segment (start 128.5 86.46) (end 130 84.96) (width 0.2) (layer "F.Cu") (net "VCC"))
 (segment (start 124.826 97.051) (end 123.1644 97.051) (width 0.2) (layer "F.Cu") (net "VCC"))
 (segment (start 128.5 90.9618) (end 128.5 86.46) (width 0.2) (layer "F.Cu") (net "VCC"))
 (segment (start 122.1134 96) (end 121 96) (width 0.2) (layer "F.Cu") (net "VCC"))
 (segment (start 126.9375 89.5375) (end 125.9 90.575) (width 0.2) (layer "F.Cu") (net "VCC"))
 (segment (start 127.8039 96.4675) (end 126.5464 97.725) (width 0.2) (layer "F.Cu") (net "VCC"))
 (segment (start 126.8167 92.2831) (end 127.1787 92.2831) (width 0.2) (layer "F.Cu") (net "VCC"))
 (segment (start 116.475 83.365) (end 118.025 83.365) (width 0.2) (layer "F.Cu") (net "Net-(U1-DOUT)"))
 (segment (start 115 84.84) (end 116.475 83.365) (width 0.2) (layer "F.Cu") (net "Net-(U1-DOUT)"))
 (segment (start 116.7492 84.2002) (end 116.9494 84) (width 0.2) (layer "F.Cu") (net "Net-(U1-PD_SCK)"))
 (segment (start 118.6942 82.7642) (end 118.025 82.095) (width 0.15) (layer "F.Cu") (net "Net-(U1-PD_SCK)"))
 (segment (start 115 87.38) (end 115 86.8382) (width 0.2) (layer "F.Cu") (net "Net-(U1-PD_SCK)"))
 (segment (start 116.7492 85.089) (end 116.7492 84.2002) (width 0.15) (layer "F.Cu") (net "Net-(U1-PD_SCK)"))
 (segment (start 115 86.8382) (end 116.7492 85.089) (width 0.2) (layer "F.Cu") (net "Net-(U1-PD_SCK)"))
 (segment (start 119.3219 83.7571) (end 119.3219 82.7642) (width 0.2) (layer "F.Cu") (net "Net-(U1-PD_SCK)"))
 (segment (start 119.3219 82.7642) (end 118.6942 82.7642) (width 0.15) (layer "F.Cu") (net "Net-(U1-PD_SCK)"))
 (segment (start 119.079 84) (end 119.3219 83.7571) (width 0.2) (layer "F.Cu") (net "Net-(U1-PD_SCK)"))
 (segment (start 116.9494 84) (end 119.079 84) (width 0.2) (layer "F.Cu") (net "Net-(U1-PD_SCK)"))
 (segment (start 127.9931 88.6592) (end 127.9931 89.8944) (width 0.2) (layer "F.Cu") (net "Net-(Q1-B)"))
 (segment (start 126.7443 87.4104) (end 127.9931 88.6592) (width 0.2) (layer "F.Cu") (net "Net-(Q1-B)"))
 (segment (start 122.975 87.175) (end 123.2104 87.4104) (width 0.2) (layer "F.Cu") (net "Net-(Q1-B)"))
 (segment (start 127.9931 89.8944) (end 126.9375 90.95) (width 0.2) (layer "F.Cu") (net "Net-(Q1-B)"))
 (segment (start 123.2104 87.4104) (end 126.7443 87.4104) (width 0.2) (layer "F.Cu") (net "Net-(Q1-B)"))
 (segment (start 121.6286 82.7642) (end 120.8642 83.5286) (width 0.15) (layer "F.Cu") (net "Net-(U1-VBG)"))
 (segment (start 122.975 82.095) (end 122.3058 82.7642) (width 0.15) (layer "F.Cu") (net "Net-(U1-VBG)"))
 (segment (start 122.55 98.0181) (end 122.55 99) (width 0.2) (layer "F.Cu") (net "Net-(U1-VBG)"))
 (segment (start 122.3058 82.7642) (end 121.6286 82.7642) (width 0.15) (layer "F.Cu") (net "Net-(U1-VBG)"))
 (via (at 122.55 98.0181) (size 0.6) (drill 0.3) (layers "F.Cu" "B.Cu") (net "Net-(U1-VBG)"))
 (via (at 120.8642 83.5286) (size 0.6) (drill 0.3) (layers "F.Cu" "B.Cu") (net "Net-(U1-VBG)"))
 (segment (start 116.4338 98.0885) (end 116.0387 97.6934) (width 0.2) (layer "B.Cu") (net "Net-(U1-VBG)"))
 (segment (start 117.0316 90.325) (end 116.1502 89.4436) (width 0.15) (layer "B.Cu") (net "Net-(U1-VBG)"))
 (segment (start 116.1502 88.5417) (end 120.8642 83.8277) (width 0.2) (layer "B.Cu") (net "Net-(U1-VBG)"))
 (segment (start 122.55 98.0181) (end 122.4796 98.0885) (width 0.2) (layer "B.Cu") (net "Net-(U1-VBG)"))
 (segment (start 116.1502 89.4436) (end 116.1502 88.5417) (width 0.15) (layer "B.Cu") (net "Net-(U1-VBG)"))
 (segment (start 116.0387 97.6934) (end 116.0387 96.9868) (width 0.2) (layer "B.Cu") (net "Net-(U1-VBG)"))
 (segment (start 116.0387 96.9868) (end 117.0316 95.9939) (width 0.2) (layer "B.Cu") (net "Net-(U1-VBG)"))
 (segment (start 122.4796 98.0885) (end 116.4338 98.0885) (width 0.2) (layer "B.Cu") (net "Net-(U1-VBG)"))
 (segment (start 117.0316 95.9939) (end 117.0316 90.325) (width 0.2) (layer "B.Cu") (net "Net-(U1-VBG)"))
 (segment (start 120.8642 83.8277) (end 120.8642 83.5286) (width 0.2) (layer "B.Cu") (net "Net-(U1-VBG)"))
 (segment (start 131.03 81.03) (end 128.85 81.03) (width 0.2) (layer "F.Cu") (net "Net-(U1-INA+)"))
 (segment (start 121.725 103.9) (end 122.5 104.675) (width 0.2) (layer "F.Cu") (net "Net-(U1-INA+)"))
 (segment (start 131.9 81.9) (end 131.03 81.03) (width 0.2) (layer "F.Cu") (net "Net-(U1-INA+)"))
 (segment (start 128.85 80.85) (end 126.5222 78.5222) (width 0.2) (layer "F.Cu") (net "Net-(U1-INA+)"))
 (segment (start 131.5 97.5) (end 131.9 97.1) (width 0.2) (layer "F.Cu") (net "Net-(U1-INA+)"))
 (segment (start 128.3358 99.4036) (end 130.2394 97.5) (width 0.2) (layer "F.Cu") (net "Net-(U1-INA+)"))
 (segment (start 126.5222 78.5222) (end 124.0078 78.5222) (width 0.2) (layer "F.Cu") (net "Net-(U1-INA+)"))
 (segment (start 121.725 101.5) (end 121.725 103.9) (width 0.2) (layer "F.Cu") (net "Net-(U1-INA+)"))
 (segment (start 122.5 104.675) (end 123.2219 105.3969) (width 0.2) (layer "F.Cu") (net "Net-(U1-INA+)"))
 (segment (start 123.2219 105.3969) (end 126.0462 105.3969) (width 0.2) (layer "F.Cu") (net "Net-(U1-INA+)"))
 (segment (start 128.85 81.03) (end 128.85 80.85) (width 0.2) (layer "F.Cu") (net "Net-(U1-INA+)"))
 (segment (start 124.0078 78.5222) (end 122.975 79.555) (width 0.2) (layer "F.Cu") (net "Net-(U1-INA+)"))
 (segment (start 126.0462 105.3969) (end 128.3358 103.1073) (width 0.2) (layer "F.Cu") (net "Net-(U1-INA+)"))
 (segment (start 130.2394 97.5) (end 131.5 97.5) (width 0.2) (layer "F.Cu") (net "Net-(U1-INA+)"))
 (segment (start 131.9 97.1) (end 131.9 81.9) (width 0.2) (layer "F.Cu") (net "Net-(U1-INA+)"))
 (segment (start 128.3358 103.1073) (end 128.3358 99.4036) (width 0.2) (layer "F.Cu") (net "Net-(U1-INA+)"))
 (segment (start 123.0983 106.9233) (end 122.5 106.325) (width 0.2) (layer "F.Cu") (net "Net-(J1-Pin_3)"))
 (segment (start 124.25 110.555) (end 123.0983 110.555) (width 0.2) (layer "F.Cu") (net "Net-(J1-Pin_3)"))
 (segment (start 123.0983 110.555) (end 123.0983 106.9233) (width 0.2) (layer "F.Cu") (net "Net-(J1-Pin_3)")))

